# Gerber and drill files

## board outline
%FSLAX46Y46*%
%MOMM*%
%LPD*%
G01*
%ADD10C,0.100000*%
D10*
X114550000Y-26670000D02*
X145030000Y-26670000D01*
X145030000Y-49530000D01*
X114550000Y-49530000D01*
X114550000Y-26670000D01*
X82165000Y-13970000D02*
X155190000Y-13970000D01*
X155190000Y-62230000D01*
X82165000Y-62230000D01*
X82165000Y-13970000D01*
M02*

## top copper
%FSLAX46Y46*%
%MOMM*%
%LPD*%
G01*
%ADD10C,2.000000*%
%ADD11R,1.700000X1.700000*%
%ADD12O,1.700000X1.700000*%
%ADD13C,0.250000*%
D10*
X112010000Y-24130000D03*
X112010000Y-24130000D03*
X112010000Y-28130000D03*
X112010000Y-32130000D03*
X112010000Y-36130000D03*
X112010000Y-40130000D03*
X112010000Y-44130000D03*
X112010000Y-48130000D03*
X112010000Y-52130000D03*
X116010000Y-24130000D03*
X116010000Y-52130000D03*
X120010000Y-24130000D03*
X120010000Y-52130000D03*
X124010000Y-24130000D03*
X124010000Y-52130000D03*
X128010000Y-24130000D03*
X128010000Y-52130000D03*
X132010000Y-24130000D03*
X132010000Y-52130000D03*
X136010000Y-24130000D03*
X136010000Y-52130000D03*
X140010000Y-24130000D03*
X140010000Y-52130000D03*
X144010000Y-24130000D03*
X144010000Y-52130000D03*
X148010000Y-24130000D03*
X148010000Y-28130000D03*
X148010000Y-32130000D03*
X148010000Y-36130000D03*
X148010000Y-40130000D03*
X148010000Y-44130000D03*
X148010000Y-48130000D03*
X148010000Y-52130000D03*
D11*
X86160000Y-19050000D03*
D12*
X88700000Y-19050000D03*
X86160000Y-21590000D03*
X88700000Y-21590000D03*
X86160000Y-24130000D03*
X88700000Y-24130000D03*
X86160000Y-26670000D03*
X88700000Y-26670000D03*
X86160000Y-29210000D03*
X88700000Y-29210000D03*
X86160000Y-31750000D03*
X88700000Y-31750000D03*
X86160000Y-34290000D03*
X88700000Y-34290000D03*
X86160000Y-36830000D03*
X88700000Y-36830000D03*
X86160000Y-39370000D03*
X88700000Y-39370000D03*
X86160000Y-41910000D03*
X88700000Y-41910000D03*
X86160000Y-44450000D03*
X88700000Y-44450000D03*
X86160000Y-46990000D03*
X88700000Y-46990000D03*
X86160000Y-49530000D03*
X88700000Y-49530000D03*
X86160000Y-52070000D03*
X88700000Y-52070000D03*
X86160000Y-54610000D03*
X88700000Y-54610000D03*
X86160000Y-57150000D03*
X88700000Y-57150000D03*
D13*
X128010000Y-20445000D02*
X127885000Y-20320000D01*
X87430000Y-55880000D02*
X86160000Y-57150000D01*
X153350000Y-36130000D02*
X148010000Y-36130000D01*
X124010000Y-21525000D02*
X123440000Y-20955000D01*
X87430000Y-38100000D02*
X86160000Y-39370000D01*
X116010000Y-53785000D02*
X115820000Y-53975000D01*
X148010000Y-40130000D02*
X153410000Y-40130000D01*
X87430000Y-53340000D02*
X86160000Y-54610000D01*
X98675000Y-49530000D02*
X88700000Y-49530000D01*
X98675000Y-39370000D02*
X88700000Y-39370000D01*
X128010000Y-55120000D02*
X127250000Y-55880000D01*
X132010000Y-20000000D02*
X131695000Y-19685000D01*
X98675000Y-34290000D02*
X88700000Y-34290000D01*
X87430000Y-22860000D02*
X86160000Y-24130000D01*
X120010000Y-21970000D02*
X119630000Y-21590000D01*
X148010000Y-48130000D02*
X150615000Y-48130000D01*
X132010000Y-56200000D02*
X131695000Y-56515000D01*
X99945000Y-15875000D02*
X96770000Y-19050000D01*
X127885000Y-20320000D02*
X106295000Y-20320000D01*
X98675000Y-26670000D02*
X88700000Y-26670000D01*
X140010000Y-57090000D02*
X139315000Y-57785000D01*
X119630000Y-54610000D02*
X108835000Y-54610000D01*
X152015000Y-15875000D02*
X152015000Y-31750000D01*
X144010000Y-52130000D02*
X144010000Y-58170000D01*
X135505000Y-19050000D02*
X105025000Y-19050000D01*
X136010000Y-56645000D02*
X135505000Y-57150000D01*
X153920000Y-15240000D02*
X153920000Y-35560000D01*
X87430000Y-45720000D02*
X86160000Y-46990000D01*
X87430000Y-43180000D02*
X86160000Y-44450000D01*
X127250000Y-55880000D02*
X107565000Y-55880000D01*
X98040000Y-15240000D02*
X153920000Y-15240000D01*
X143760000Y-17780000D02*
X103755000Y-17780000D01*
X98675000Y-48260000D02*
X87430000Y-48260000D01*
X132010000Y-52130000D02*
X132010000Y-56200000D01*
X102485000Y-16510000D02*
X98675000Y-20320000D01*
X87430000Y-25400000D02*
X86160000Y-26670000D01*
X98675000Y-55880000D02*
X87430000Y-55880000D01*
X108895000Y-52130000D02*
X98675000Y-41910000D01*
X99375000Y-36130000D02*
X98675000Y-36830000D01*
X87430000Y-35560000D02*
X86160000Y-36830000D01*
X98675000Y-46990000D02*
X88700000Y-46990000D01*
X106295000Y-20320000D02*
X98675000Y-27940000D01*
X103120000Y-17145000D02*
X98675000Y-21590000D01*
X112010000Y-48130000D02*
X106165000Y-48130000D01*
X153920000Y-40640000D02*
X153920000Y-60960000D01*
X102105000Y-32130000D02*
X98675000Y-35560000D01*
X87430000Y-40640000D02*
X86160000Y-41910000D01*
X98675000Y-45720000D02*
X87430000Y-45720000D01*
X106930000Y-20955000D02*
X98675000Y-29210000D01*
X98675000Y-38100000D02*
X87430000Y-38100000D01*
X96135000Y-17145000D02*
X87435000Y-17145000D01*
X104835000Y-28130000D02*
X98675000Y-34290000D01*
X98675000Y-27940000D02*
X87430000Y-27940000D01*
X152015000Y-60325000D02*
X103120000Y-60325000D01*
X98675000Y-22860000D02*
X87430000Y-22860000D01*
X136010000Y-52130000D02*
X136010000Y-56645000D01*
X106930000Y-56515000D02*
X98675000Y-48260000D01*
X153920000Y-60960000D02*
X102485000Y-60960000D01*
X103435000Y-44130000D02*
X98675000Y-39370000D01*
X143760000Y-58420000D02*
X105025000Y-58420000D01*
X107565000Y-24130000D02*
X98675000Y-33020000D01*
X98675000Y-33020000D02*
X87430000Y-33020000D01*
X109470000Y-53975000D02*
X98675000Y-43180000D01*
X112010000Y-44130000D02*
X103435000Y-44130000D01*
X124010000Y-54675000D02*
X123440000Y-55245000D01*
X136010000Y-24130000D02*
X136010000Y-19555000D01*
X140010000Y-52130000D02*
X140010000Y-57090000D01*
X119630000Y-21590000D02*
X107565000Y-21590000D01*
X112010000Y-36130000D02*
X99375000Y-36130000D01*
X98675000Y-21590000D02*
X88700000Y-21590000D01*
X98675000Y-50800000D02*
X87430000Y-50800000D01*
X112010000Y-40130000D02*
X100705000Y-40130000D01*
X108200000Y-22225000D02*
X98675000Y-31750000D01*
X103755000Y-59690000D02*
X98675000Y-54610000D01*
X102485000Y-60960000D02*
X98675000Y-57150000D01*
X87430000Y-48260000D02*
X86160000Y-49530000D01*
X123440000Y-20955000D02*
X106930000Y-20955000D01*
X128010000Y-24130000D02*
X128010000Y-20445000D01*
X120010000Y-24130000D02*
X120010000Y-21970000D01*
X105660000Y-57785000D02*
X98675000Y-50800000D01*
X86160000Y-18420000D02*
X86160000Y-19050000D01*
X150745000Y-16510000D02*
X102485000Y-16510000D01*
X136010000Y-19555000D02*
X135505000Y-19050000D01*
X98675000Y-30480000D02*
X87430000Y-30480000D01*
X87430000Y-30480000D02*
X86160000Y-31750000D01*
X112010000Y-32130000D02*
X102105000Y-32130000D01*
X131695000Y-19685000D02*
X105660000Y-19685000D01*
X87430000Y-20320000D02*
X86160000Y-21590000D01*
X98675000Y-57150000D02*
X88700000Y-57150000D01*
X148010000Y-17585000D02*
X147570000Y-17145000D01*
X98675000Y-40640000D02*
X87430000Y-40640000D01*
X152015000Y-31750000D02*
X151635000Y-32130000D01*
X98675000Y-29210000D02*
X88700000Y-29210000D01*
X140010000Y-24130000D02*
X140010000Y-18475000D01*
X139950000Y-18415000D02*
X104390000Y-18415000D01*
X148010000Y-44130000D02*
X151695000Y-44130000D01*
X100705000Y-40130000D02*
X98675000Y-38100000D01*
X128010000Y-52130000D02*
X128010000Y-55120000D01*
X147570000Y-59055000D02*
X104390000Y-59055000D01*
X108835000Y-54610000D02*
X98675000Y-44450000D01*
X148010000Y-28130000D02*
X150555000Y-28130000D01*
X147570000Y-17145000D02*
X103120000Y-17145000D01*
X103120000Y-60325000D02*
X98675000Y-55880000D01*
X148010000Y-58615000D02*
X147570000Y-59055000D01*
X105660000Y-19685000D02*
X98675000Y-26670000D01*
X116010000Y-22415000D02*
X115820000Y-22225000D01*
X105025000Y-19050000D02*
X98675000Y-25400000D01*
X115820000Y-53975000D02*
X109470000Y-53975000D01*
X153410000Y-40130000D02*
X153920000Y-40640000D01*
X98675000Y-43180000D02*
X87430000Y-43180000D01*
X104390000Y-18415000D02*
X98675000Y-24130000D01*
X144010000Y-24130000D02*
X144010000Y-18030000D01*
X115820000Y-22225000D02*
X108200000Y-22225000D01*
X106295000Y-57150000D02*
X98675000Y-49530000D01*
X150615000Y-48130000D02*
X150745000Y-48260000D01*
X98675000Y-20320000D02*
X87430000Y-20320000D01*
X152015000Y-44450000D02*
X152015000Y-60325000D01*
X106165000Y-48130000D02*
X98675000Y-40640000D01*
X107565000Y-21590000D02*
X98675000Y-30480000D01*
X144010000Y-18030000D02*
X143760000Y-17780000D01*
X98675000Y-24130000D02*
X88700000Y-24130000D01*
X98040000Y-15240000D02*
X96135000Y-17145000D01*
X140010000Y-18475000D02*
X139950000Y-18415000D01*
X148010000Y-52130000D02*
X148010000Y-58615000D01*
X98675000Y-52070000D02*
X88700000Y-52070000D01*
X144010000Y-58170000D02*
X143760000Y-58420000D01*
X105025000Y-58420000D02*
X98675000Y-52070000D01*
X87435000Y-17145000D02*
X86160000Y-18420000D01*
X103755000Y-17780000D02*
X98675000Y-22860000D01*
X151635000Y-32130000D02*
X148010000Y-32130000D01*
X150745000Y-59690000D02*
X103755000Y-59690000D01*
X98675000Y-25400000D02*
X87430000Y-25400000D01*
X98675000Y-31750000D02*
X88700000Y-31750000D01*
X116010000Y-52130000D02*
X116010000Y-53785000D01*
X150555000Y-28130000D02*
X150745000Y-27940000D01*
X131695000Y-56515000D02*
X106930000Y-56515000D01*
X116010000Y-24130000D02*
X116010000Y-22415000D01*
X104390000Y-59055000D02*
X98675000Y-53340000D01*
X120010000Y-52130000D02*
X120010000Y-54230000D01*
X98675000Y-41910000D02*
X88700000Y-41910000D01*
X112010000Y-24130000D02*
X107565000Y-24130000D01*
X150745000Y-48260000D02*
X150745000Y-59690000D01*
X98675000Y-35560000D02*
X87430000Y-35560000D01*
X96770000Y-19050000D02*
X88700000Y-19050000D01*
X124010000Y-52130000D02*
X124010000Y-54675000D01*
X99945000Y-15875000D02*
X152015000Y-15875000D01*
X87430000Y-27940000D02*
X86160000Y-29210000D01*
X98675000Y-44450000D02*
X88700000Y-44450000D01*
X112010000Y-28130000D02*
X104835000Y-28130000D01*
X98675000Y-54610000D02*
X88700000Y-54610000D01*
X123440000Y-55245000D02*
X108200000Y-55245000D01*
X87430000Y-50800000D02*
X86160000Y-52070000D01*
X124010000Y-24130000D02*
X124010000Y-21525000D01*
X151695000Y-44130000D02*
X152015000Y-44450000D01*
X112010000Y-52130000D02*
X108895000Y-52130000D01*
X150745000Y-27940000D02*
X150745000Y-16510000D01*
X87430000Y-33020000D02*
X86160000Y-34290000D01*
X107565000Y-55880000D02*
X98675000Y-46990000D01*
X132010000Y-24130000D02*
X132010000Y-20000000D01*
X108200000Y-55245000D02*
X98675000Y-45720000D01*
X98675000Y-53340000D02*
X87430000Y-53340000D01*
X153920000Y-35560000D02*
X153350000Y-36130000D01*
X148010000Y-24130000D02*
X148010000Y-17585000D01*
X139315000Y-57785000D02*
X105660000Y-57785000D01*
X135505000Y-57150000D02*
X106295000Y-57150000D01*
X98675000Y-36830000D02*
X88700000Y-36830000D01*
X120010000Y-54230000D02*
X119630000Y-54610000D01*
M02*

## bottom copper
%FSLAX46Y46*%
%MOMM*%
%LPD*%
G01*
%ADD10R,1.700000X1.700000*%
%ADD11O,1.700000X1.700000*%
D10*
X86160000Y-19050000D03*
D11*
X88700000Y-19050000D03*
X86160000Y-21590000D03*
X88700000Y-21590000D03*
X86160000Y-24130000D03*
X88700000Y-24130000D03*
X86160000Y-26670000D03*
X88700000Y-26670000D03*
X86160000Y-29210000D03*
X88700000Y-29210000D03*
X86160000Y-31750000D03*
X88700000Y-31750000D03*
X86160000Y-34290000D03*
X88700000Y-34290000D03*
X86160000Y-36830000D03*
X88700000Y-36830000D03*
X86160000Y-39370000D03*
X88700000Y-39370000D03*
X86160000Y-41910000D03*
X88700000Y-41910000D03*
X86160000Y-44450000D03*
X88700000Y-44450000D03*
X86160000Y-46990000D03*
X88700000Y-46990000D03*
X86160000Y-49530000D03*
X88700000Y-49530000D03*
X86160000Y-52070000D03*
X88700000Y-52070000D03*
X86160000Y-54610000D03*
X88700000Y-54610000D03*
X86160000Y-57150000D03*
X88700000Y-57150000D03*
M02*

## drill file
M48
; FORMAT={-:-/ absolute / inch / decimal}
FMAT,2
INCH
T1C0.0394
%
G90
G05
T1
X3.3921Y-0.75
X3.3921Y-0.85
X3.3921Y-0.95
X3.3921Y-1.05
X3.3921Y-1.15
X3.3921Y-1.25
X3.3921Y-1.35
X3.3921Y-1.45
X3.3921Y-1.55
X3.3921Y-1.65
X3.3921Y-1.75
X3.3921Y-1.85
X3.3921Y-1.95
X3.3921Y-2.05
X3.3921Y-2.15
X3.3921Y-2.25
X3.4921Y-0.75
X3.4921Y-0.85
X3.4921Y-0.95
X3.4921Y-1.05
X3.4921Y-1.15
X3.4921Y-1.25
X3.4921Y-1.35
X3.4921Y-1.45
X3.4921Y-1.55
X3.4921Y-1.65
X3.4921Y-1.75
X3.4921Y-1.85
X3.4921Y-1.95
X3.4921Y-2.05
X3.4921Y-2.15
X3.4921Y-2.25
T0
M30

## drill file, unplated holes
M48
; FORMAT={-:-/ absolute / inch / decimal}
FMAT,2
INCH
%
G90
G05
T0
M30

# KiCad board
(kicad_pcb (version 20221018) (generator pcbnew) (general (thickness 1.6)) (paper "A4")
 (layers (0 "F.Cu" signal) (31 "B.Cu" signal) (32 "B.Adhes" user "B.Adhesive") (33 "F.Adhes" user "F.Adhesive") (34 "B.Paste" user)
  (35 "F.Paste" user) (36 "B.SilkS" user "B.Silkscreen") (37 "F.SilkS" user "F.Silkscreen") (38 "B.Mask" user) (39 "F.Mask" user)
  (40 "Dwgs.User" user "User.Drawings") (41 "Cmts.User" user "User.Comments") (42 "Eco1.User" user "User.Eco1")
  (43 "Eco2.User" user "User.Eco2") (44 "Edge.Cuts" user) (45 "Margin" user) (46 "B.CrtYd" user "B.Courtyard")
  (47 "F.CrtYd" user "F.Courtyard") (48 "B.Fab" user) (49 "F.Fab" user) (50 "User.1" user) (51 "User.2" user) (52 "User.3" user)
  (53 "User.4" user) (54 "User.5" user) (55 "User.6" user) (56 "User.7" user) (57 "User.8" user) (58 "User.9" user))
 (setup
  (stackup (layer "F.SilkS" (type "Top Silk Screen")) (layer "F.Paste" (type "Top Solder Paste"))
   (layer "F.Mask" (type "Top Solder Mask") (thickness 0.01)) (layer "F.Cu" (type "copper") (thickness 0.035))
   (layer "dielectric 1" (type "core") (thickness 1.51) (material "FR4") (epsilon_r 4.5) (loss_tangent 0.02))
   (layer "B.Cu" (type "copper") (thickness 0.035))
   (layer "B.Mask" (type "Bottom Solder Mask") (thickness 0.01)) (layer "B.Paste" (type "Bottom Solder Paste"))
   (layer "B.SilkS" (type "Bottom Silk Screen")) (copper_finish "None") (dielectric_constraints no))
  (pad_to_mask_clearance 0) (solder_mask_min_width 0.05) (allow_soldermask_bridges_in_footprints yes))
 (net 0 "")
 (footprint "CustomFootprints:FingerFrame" (layer "F.Cu") (at 112.01 24.13)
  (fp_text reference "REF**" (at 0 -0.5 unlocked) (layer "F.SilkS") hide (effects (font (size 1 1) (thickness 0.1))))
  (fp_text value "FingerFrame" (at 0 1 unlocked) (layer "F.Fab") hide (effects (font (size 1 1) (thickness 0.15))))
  (pad "1" smd circle (at 0 0) (size 2 2) (layers "F.Cu" "F.Paste" "F.Mask"))
  (pad "1" smd circle (at 0 0) (size 2 2) (layers "F.Cu" "F.Paste" "F.Mask"))
  (pad "1" smd circle (at 0 4) (size 2 2) (layers "F.Cu" "F.Paste" "F.Mask"))
  (pad "1" smd circle (at 0 8) (size 2 2) (layers "F.Cu" "F.Paste" "F.Mask"))
  (pad "1" smd circle (at 0 12) (size 2 2) (layers "F.Cu" "F.Paste" "F.Mask"))
  (pad "1" smd circle (at 0 16) (size 2 2) (layers "F.Cu" "F.Paste" "F.Mask"))
  (pad "1" smd circle (at 0 20) (size 2 2) (layers "F.Cu" "F.Paste" "F.Mask"))
  (pad "1" smd circle (at 0 24) (size 2 2) (layers "F.Cu" "F.Paste" "F.Mask"))
  (pad "1" smd circle (at 0 28) (size 2 2) (layers "F.Cu" "F.Paste" "F.Mask"))
  (pad "1" smd circle (at 4 0) (size 2 2) (layers "F.Cu" "F.Paste" "F.Mask"))
  (pad "1" smd circle (at 4 28) (size 2 2) (layers "F.Cu" "F.Paste" "F.Mask"))
  (pad "1" smd circle (at 8 0) (size 2 2) (layers "F.Cu" "F.Paste" "F.Mask"))
  (pad "1" smd circle (at 8 28) (size 2 2) (layers "F.Cu" "F.Paste" "F.Mask"))
  (pad "1" smd circle (at 12 0) (size 2 2) (layers "F.Cu" "F.Paste" "F.Mask"))
  (pad "1" smd circle (at 12 28) (size 2 2) (layers "F.Cu" "F.Paste" "F.Mask"))
  (pad "1" smd circle (at 16 0) (size 2 2) (layers "F.Cu" "F.Paste" "F.Mask"))
  (pad "1" smd circle (at 16 28) (size 2 2) (layers "F.Cu" "F.Paste" "F.Mask"))
  (pad "1" smd circle (at 20 0) (size 2 2) (layers "F.Cu" "F.Paste" "F.Mask"))
  (pad "1" smd circle (at 20 28) (size 2 2) (layers "F.Cu" "F.Paste" "F.Mask"))
  (pad "1" smd circle (at 24 0) (size 2 2) (layers "F.Cu" "F.Paste" "F.Mask"))
  (pad "1" smd circle (at 24 28) (size 2 2) (layers "F.Cu" "F.Paste" "F.Mask"))
  (pad "1" smd circle (at 28 0) (size 2 2) (layers "F.Cu" "F.Paste" "F.Mask"))
  (pad "1" smd circle (at 28 28) (size 2 2) (layers "F.Cu" "F.Paste" "F.Mask"))
  (pad "1" smd circle (at 32 0) (size 2 2) (layers "F.Cu" "F.Paste" "F.Mask"))
  (pad "1" smd circle (at 32 28) (size 2 2) (layers "F.Cu" "F.Paste" "F.Mask"))
  (pad "1" smd circle (at 36 0) (size 2 2) (layers "F.Cu" "F.Paste" "F.Mask"))
  (pad "1" smd circle (at 36 4) (size 2 2) (layers "F.Cu" "F.Paste" "F.Mask"))
  (pad "1" smd circle (at 36 8) (size 2 2) (layers "F.Cu" "F.Paste" "F.Mask"))
  (pad "1" smd circle (at 36 12) (size 2 2) (layers "F.Cu" "F.Paste" "F.Mask"))
  (pad "1" smd circle (at 36 16) (size 2 2) (layers "F.Cu" "F.Paste" "F.Mask"))
  (pad "1" smd circle (at 36 20) (size 2 2) (layers "F.Cu" "F.Paste" "F.Mask"))
  (pad "1" smd circle (at 36 24) (size 2 2) (layers "F.Cu" "F.Paste" "F.Mask"))
  (pad "1" smd circle (at 36 28) (size 2 2) (layers "F.Cu" "F.Paste" "F.Mask")))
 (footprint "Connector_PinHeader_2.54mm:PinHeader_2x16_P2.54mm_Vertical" (layer "F.Cu") (at 86.16 19.05)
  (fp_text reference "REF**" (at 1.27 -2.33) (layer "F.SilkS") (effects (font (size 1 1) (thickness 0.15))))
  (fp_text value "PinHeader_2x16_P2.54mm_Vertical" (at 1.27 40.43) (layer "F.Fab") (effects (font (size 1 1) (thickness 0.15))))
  (pad "1" thru_hole rect (at 0 0) (size 1.7 1.7) (drill 1) (layers "*.Cu" "*.Mask"))
  (pad "2" thru_hole oval (at 2.54 0) (size 1.7 1.7) (drill 1) (layers "*.Cu" "*.Mask"))
  (pad "3" thru_hole oval (at 0 2.54) (size 1.7 1.7) (drill 1) (layers "*.Cu" "*.Mask"))
  (pad "4" thru_hole oval (at 2.54 2.54) (size 1.7 1.7) (drill 1) (layers "*.Cu" "*.Mask"))
  (pad "5" thru_hole oval (at 0 5.08) (size 1.7 1.7) (drill 1) (layers "*.Cu" "*.Mask"))
  (pad "6" thru_hole oval (at 2.54 5.08) (size 1.7 1.7) (drill 1) (layers "*.Cu" "*.Mask"))
  (pad "7" thru_hole oval (at 0 7.62) (size 1.7 1.7) (drill 1) (layers "*.Cu" "*.Mask"))
  (pad "8" thru_hole oval (at 2.54 7.62) (size 1.7 1.7) (drill 1) (layers "*.Cu" "*.Mask"))
  (pad "9" thru_hole oval (at 0 10.16) (size 1.7 1.7) (drill 1) (layers "*.Cu" "*.Mask"))
  (pad "10" thru_hole oval (at 2.54 10.16) (size 1.7 1.7) (drill 1) (layers "*.Cu" "*.Mask"))
  (pad "11" thru_hole oval (at 0 12.7) (size 1.7 1.7) (drill 1) (layers "*.Cu" "*.Mask"))
  (pad "12" thru_hole oval (at 2.54 12.7) (size 1.7 1.7) (drill 1) (layers "*.Cu" "*.Mask"))
  (pad "13" thru_hole oval (at 0 15.24) (size 1.7 1.7) (drill 1) (layers "*.Cu" "*.Mask"))
  (pad "14" thru_hole oval (at 2.54 15.24) (size 1.7 1.7) (drill 1) (layers "*.Cu" "*.Mask"))
  (pad "15" thru_hole oval (at 0 17.78) (size 1.7 1.7) (drill 1) (layers "*.Cu" "*.Mask"))
  (pad "16" thru_hole oval (at 2.54 17.78) (size 1.7 1.7) (drill 1) (layers "*.Cu" "*.Mask"))
  (pad "17" thru_hole oval (at 0 20.32) (size 1.7 1.7) (drill 1) (layers "*.Cu" "*.Mask"))
  (pad "18" thru_hole oval (at 2.54 20.32) (size 1.7 1.7) (drill 1) (layers "*.Cu" "*.Mask"))
  (pad "19" thru_hole oval (at 0 22.86) (size 1.7 1.7) (drill 1) (layers "*.Cu" "*.Mask"))
  (pad "20" thru_hole oval (at 2.54 22.86) (size 1.7 1.7) (drill 1) (layers "*.Cu" "*.Mask"))
  (pad "21" thru_hole oval (at 0 25.4) (size 1.7 1.7) (drill 1) (layers "*.Cu" "*.Mask"))
  (pad "22" thru_hole oval (at 2.54 25.4) (size 1.7 1.7) (drill 1) (layers "*.Cu" "*.Mask"))
  (pad "23" thru_hole oval (at 0 27.94) (size 1.7 1.7) (drill 1) (layers "*.Cu" "*.Mask"))
  (pad "24" thru_hole oval (at 2.54 27.94) (size 1.7 1.7) (drill 1) (layers "*.Cu" "*.Mask"))
  (pad "25" thru_hole oval (at 0 30.48) (size 1.7 1.7) (drill 1) (layers "*.Cu" "*.Mask"))
  (pad "26" thru_hole oval (at 2.54 30.48) (size 1.7 1.7) (drill 1) (layers "*.Cu" "*.Mask"))
  (pad "27" thru_hole oval (at 0 33.02) (size 1.7 1.7) (drill 1) (layers "*.Cu" "*.Mask"))
  (pad "28" thru_hole oval (at 2.54 33.02) (size 1.7 1.7) (drill 1) (layers "*.Cu" "*.Mask"))
  (pad "29" thru_hole oval (at 0 35.56) (size 1.7 1.7) (drill 1) (layers "*.Cu" "*.Mask"))
  (pad "30" thru_hole oval (at 2.54 35.56) (size 1.7 1.7) (drill 1) (layers "*.Cu" "*.Mask"))
  (pad "31" thru_hole oval (at 0 38.1) (size 1.7 1.7) (drill 1) (layers "*.Cu" "*.Mask"))
  (pad "32" thru_hole oval (at 2.54 38.1) (size 1.7 1.7) (drill 1) (layers "*.Cu" "*.Mask")))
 (gr_rect (start 114.55 26.67) (end 145.03 49.53) (stroke (width 0.1) (type default)) (fill none) (layer "Edge.Cuts"))
 (gr_rect (start 82.165 13.97) (end 155.19 62.23) (stroke (width 0.1) (type default)) (fill none) (layer "Edge.Cuts"))
 (segment (start 128.01 20.445) (end 127.885 20.32) (width 0.25) (layer "F.Cu") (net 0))
 (segment (start 87.43 55.88) (end 86.16 57.15) (width 0.25) (layer "F.Cu") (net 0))
 (segment (start 153.35 36.13) (end 148.01 36.13) (width 0.25) (layer "F.Cu") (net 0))
 (segment (start 124.01 21.525) (end 123.44 20.955) (width 0.25) (layer "F.Cu") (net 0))
 (segment (start 87.43 38.1) (end 86.16 39.37) (width 0.25) (layer "F.Cu") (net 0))
 (segment (start 116.01 53.785) (end 115.82 53.975) (width 0.25) (layer "F.Cu") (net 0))
 (segment (start 148.01 40.13) (end 153.41 40.13) (width 0.25) (layer "F.Cu") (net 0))
 (segment (start 87.43 53.34) (end 86.16 54.61) (width 0.25) (layer "F.Cu") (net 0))
 (segment (start 98.675 49.53) (end 88.7 49.53) (width 0.25) (layer "F.Cu") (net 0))
 (segment (start 98.675 39.37) (end 88.7 39.37) (width 0.25) (layer "F.Cu") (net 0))
 (segment (start 128.01 55.12) (end 127.25 55.88) (width 0.25) (layer "F.Cu") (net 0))
 (segment (start 132.01 20) (end 131.695 19.685) (width 0.25) (layer "F.Cu") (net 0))
 (segment (start 98.675 34.29) (end 88.7 34.29) (width 0.25) (layer "F.Cu") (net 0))
 (segment (start 87.43 22.86) (end 86.16 24.13) (width 0.25) (layer "F.Cu") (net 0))
 (segment (start 120.01 21.97) (end 119.63 21.59) (width 0.25) (layer "F.Cu") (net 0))
 (segment (start 148.01 48.13) (end 150.615 48.13) (width 0.25) (layer "F.Cu") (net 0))
 (segment (start 132.01 56.2) (end 131.695 56.515) (width 0.25) (layer "F.Cu") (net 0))
 (segment (start 99.945 15.875) (end 96.77 19.05) (width 0.25) (layer "F.Cu") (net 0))
 (segment (start 127.885 20.32) (end 106.295 20.32) (width 0.25) (layer "F.Cu") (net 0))
 (segment (start 98.675 26.67) (end 88.7 26.67) (width 0.25) (layer "F.Cu") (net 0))
 (segment (start 140.01 57.09) (end 139.315 57.785) (width 0.25) (layer "F.Cu") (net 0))
 (segment (start 119.63 54.61) (end 108.835 54.61) (width 0.25) (layer "F.Cu") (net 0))
 (segment (start 152.015 15.875) (end 152.015 31.75) (width 0.25) (layer "F.Cu") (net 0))
 (segment (start 144.01 52.13) (end 144.01 58.17) (width 0.25) (layer "F.Cu") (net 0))
 (segment (start 135.505 19.05) (end 105.025 19.05) (width 0.25) (layer "F.Cu") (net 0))
 (segment (start 136.01 56.645) (end 135.505 57.15) (width 0.25) (layer "F.Cu") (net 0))
 (segment (start 153.92 15.24) (end 153.92 35.56) (width 0.25) (layer "F.Cu") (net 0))
 (segment (start 87.43 45.72) (end 86.16 46.99) (width 0.25) (layer "F.Cu") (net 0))
 (segment (start 87.43 43.18) (end 86.16 44.45) (width 0.25) (layer "F.Cu") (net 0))
 (segment (start 127.25 55.88) (end 107.565 55.88) (width 0.25) (layer "F.Cu") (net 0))
 (segment (start 98.04 15.24) (end 153.92 15.24) (width 0.25) (layer "F.Cu") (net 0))
 (segment (start 143.76 17.78) (end 103.755 17.78) (width 0.25) (layer "F.Cu") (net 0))
 (segment (start 98.675 48.26) (end 87.43 48.26) (width 0.25) (layer "F.Cu") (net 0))
 (segment (start 132.01 52.13) (end 132.01 56.2) (width 0.25) (layer "F.Cu") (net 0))
 (segment (start 102.485 16.51) (end 98.675 20.32) (width 0.25) (layer "F.Cu") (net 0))
 (segment (start 87.43 25.4) (end 86.16 26.67) (width 0.25) (layer "F.Cu") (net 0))
 (segment (start 98.675 55.88) (end 87.43 55.88) (width 0.25) (layer "F.Cu") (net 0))
 (segment (start 108.895 52.13) (end 98.675 41.91) (width 0.25) (layer "F.Cu") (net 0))
 (segment (start 99.375 36.13) (end 98.675 36.83) (width 0.25) (layer "F.Cu") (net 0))
 (segment (start 87.43 35.56) (end 86.16 36.83) (width 0.25) (layer "F.Cu") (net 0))
 (segment (start 98.675 46.99) (end 88.7 46.99) (width 0.25) (layer "F.Cu") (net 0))
 (segment (start 106.295 20.32) (end 98.675 27.94) (width 0.25) (layer "F.Cu") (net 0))
 (segment (start 103.12 17.145) (end 98.675 21.59) (width 0.25) (layer "F.Cu") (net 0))
 (segment (start 112.01 48.13) (end 106.165 48.13) (width 0.25) (layer "F.Cu") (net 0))
 (segment (start 153.92 40.64) (end 153.92 60.96) (width 0.25) (layer "F.Cu") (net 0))
 (segment (start 102.105 32.13) (end 98.675 35.56) (width 0.25) (layer "F.Cu") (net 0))
 (segment (start 87.43 40.64) (end 86.16 41.91) (width 0.25) (layer "F.Cu") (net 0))
 (segment (start 98.675 45.72) (end 87.43 45.72) (width 0.25) (layer "F.Cu") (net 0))
 (segment (start 106.93 20.955) (end 98.675 29.21) (width 0.25) (layer "F.Cu") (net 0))
 (segment (start 98.675 38.1) (end 87.43 38.1) (width 0.25) (layer "F.Cu") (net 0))
 (segment (start 96.135 17.145) (end 87.435 17.145) (width 0.25) (layer "F.Cu") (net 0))
 (segment (start 104.835 28.13) (end 98.675 34.29) (width 0.25) (layer "F.Cu") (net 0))
 (segment (start 98.675 27.94) (end 87.43 27.94) (width 0.25) (layer "F.Cu") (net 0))
 (segment (start 152.015 60.325) (end 103.12 60.325) (width 0.25) (layer "F.Cu") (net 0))
 (segment (start 98.675 22.86) (end 87.43 22.86) (width 0.25) (layer "F.Cu") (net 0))
 (segment (start 136.01 52.13) (end 136.01 56.645) (width 0.25) (layer "F.Cu") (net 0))
 (segment (start 106.93 56.515) (end 98.675 48.26) (width 0.25) (layer "F.Cu") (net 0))
 (segment (start 153.92 60.96) (end 102.485 60.96) (width 0.25) (layer "F.Cu") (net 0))
 (segment (start 103.435 44.13) (end 98.675 39.37) (width 0.25) (layer "F.Cu") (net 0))
 (segment (start 143.76 58.42) (end 105.025 58.42) (width 0.25) (layer "F.Cu") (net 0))
 (segment (start 107.565 24.13) (end 98.675 33.02) (width 0.25) (layer "F.Cu") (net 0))
 (segment (start 98.675 33.02) (end 87.43 33.02) (width 0.25) (layer "F.Cu") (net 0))
 (segment (start 109.47 53.975) (end 98.675 43.18) (width 0.25) (layer "F.Cu") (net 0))
 (segment (start 112.01 44.13) (end 103.435 44.13) (width 0.25) (layer "F.Cu") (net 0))
 (segment (start 124.01 54.675) (end 123.44 55.245) (width 0.25) (layer "F.Cu") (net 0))
 (segment (start 136.01 24.13) (end 136.01 19.555) (width 0.25) (layer "F.Cu") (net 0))
 (segment (start 140.01 52.13) (end 140.01 57.09) (width 0.25) (layer "F.Cu") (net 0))
 (segment (start 119.63 21.59) (end 107.565 21.59) (width 0.25) (layer "F.Cu") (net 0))
 (segment (start 112.01 36.13) (end 99.375 36.13) (width 0.25) (layer "F.Cu") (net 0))
 (segment (start 98.675 21.59) (end 88.7 21.59) (width 0.25) (layer "F.Cu") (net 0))
 (segment (start 98.675 50.8) (end 87.43 50.8) (width 0.25) (layer "F.Cu") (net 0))
 (segment (start 112.01 40.13) (end 100.705 40.13) (width 0.25) (layer "F.Cu") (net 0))
 (segment (start 108.2 22.225) (end 98.675 31.75) (width 0.25) (layer "F.Cu") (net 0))
 (segment (start 103.755 59.69) (end 98.675 54.61) (width 0.25) (layer "F.Cu") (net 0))
 (segment (start 102.485 60.96) (end 98.675 57.15) (width 0.25) (layer "F.Cu") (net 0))
 (segment (start 87.43 48.26) (end 86.16 49.53) (width 0.25) (layer "F.Cu") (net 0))
 (segment (start 123.44 20.955) (end 106.93 20.955) (width 0.25) (layer "F.Cu") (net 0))
 (segment (start 128.01 24.13) (end 128.01 20.445) (width 0.25) (layer "F.Cu") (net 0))
 (segment (start 120.01 24.13) (end 120.01 21.97) (width 0.25) (layer "F.Cu") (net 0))
 (segment (start 105.66 57.785) (end 98.675 50.8) (width 0.25) (layer "F.Cu") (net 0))
 (segment (start 86.16 18.42) (end 86.16 19.05) (width 0.25) (layer "F.Cu") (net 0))
 (segment (start 150.745 16.51) (end 102.485 16.51) (width 0.25) (layer "F.Cu") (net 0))
 (segment (start 136.01 19.555) (end 135.505 19.05) (width 0.25) (layer "F.Cu") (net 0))
 (segment (start 98.675 30.48) (end 87.43 30.48) (width 0.25) (layer "F.Cu") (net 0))
 (segment (start 87.43 30.48) (end 86.16 31.75) (width 0.25) (layer "F.Cu") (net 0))
 (segment (start 112.01 32.13) (end 102.105 32.13) (width 0.25) (layer "F.Cu") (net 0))
 (segment (start 131.695 19.685) (end 105.66 19.685) (width 0.25) (layer "F.Cu") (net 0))
 (segment (start 87.43 20.32) (end 86.16 21.59) (width 0.25) (layer "F.Cu") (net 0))
 (segment (start 98.675 57.15) (end 88.7 57.15) (width 0.25) (layer "F.Cu") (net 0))
 (segment (start 148.01 17.585) (end 147.57 17.145) (width 0.25) (layer "F.Cu") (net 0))
 (segment (start 98.675 40.64) (end 87.43 40.64) (width 0.25) (layer "F.Cu") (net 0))
 (segment (start 152.015 31.75) (end 151.635 32.13) (width 0.25) (layer "F.Cu") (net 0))
 (segment (start 98.675 29.21) (end 88.7 29.21) (width 0.25) (layer "F.Cu") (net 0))
 (segment (start 140.01 24.13) (end 140.01 18.475) (width 0.25) (layer "F.Cu") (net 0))
 (segment (start 139.95 18.415) (end 104.39 18.415) (width 0.25) (layer "F.Cu") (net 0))
 (segment (start 148.01 44.13) (end 151.695 44.13) (width 0.25) (layer "F.Cu") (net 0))
 (segment (start 100.705 40.13) (end 98.675 38.1) (width 0.25) (layer "F.Cu") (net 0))
 (segment (start 128.01 52.13) (end 128.01 55.12) (width 0.25) (layer "F.Cu") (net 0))
 (segment (start 147.57 59.055) (end 104.39 59.055) (width 0.25) (layer "F.Cu") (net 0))
 (segment (start 108.835 54.61) (end 98.675 44.45) (width 0.25) (layer "F.Cu") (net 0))
 (segment (start 148.01 28.13) (end 150.555 28.13) (width 0.25) (layer "F.Cu") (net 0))
 (segment (start 147.57 17.145) (end 103.12 17.145) (width 0.25) (layer "F.Cu") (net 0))
 (segment (start 103.12 60.325) (end 98.675 55.88) (width 0.25) (layer "F.Cu") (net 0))
 (segment (start 148.01 58.615) (end 147.57 59.055) (width 0.25) (layer "F.Cu") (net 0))
 (segment (start 105.66 19.685) (end 98.675 26.67) (width 0.25) (layer "F.Cu") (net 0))
 (segment (start 116.01 22.415) (end 115.82 22.225) (width 0.25) (layer "F.Cu") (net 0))
 (segment (start 105.025 19.05) (end 98.675 25.4) (width 0.25) (layer "F.Cu") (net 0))
 (segment (start 115.82 53.975) (end 109.47 53.975) (width 0.25) (layer "F.Cu") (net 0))
 (segment (start 153.41 40.13) (end 153.92 40.64) (width 0.25) (layer "F.Cu") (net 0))
 (segment (start 98.675 43.18) (end 87.43 43.18) (width 0.25) (layer "F.Cu") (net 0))
 (segment (start 104.39 18.415) (end 98.675 24.13) (width 0.25) (layer "F.Cu") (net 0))
 (segment (start 144.01 24.13) (end 144.01 18.03) (width 0.25) (layer "F.Cu") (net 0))
 (segment (start 115.82 22.225) (end 108.2 22.225) (width 0.25) (layer "F.Cu") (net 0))
 (segment (start 106.295 57.15) (end 98.675 49.53) (width 0.25) (layer "F.Cu") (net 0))
 (segment (start 150.615 48.13) (end 150.745 48.26) (width 0.25) (layer "F.Cu") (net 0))
 (segment (start 98.675 20.32) (end 87.43 20.32) (width 0.25) (layer "F.Cu") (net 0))
 (segment (start 152.015 44.45) (end 152.015 60.325) (width 0.25) (layer "F.Cu") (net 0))
 (segment (start 106.165 48.13) (end 98.675 40.64) (width 0.25) (layer "F.Cu") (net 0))
 (segment (start 107.565 21.59) (end 98.675 30.48) (width 0.25) (layer "F.Cu") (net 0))
 (segment (start 144.01 18.03) (end 143.76 17.78) (width 0.25) (layer "F.Cu") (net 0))
 (segment (start 98.675 24.13) (end 88.7 24.13) (width 0.25) (layer "F.Cu") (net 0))
 (segment (start 98.04 15.24) (end 96.135 17.145) (width 0.25) (layer "F.Cu") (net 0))
 (segment (start 140.01 18.475) (end 139.95 18.415) (width 0.25) (layer "F.Cu") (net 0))
 (segment (start 148.01 52.13) (end 148.01 58.615) (width 0.25) (layer "F.Cu") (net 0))
 (segment (start 98.675 52.07) (end 88.7 52.07) (width 0.25) (layer "F.Cu") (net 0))
 (segment (start 144.01 58.17) (end 143.76 58.42) (width 0.25) (layer "F.Cu") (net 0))
 (segment (start 105.025 58.42) (end 98.675 52.07) (width 0.25) (layer "F.Cu") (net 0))
 (segment (start 87.435 17.145) (end 86.16 18.42) (width 0.25) (layer "F.Cu") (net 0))
 (segment (start 103.755 17.78) (end 98.675 22.86) (width 0.25) (layer "F.Cu") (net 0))
 (segment (start 151.635 32.13) (end 148.01 32.13) (width 0.25) (layer "F.Cu") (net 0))
 (segment (start 150.745 59.69) (end 103.755 59.69) (width 0.25) (layer "F.Cu") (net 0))
 (segment (start 98.675 25.4) (end 87.43 25.4) (width 0.25) (layer "F.Cu") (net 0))
 (segment (start 98.675 31.75) (end 88.7 31.75) (width 0.25) (layer "F.Cu") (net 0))
 (segment (start 116.01 52.13) (end 116.01 53.785) (width 0.25) (layer "F.Cu") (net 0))
 (segment (start 150.555 28.13) (end 150.745 27.94) (width 0.25) (layer "F.Cu") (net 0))
 (segment (start 131.695 56.515) (end 106.93 56.515) (width 0.25) (layer "F.Cu") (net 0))
 (segment (start 116.01 24.13) (end 116.01 22.415) (width 0.25) (layer "F.Cu") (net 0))
 (segment (start 104.39 59.055) (end 98.675 53.34) (width 0.25) (layer "F.Cu") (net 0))
 (segment (start 120.01 52.13) (end 120.01 54.23) (width 0.25) (layer "F.Cu") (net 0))
 (segment (start 98.675 41.91) (end 88.7 41.91) (width 0.25) (layer "F.Cu") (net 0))
 (segment (start 112.01 24.13) (end 107.565 24.13) (width 0.25) (layer "F.Cu") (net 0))
 (segment (start 150.745 48.26) (end 150.745 59.69) (width 0.25) (layer "F.Cu") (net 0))
 (segment (start 98.675 35.56) (end 87.43 35.56) (width 0.25) (layer "F.Cu") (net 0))
 (segment (start 96.77 19.05) (end 88.7 19.05) (width 0.25) (layer "F.Cu") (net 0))
 (segment (start 124.01 52.13) (end 124.01 54.675) (width 0.25) (layer "F.Cu") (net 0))
 (segment (start 99.945 15.875) (end 152.015 15.875) (width 0.25) (layer "F.Cu") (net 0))
 (segment (start 87.43 27.94) (end 86.16 29.21) (width 0.25) (layer "F.Cu") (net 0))
 (segment (start 98.675 44.45) (end 88.7 44.45) (width 0.25) (layer "F.Cu") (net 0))
 (segment (start 112.01 28.13) (end 104.835 28.13) (width 0.25) (layer "F.Cu") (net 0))
 (segment (start 98.675 54.61) (end 88.7 54.61) (width 0.25) (layer "F.Cu") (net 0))
 (segment (start 123.44 55.245) (end 108.2 55.245) (width 0.25) (layer "F.Cu") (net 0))
 (segment (start 87.43 50.8) (end 86.16 52.07) (width 0.25) (layer "F.Cu") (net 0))
 (segment (start 124.01 24.13) (end 124.01 21.525) (width 0.25) (layer "F.Cu") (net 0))
 (segment (start 151.695 44.13) (end 152.015 44.45) (width 0.25) (layer "F.Cu") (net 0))
 (segment (start 112.01 52.13) (end 108.895 52.13) (width 0.25) (layer "F.Cu") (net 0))
 (segment (start 150.745 27.94) (end 150.745 16.51) (width 0.25) (layer "F.Cu") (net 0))
 (segment (start 87.43 33.02) (end 86.16 34.29) (width 0.25) (layer "F.Cu") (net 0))
 (segment (start 107.565 55.88) (end 98.675 46.99) (width 0.25) (layer "F.Cu") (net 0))
 (segment (start 132.01 24.13) (end 132.01 20) (width 0.25) (layer "F.Cu") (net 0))
 (segment (start 108.2 55.245) (end 98.675 45.72) (width 0.25) (layer "F.Cu") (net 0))
 (segment (start 98.675 53.34) (end 87.43 53.34) (width 0.25) (layer "F.Cu") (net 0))
 (segment (start 153.92 35.56) (end 153.35 36.13) (width 0.25) (layer "F.Cu") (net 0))
 (segment (start 148.01 24.13) (end 148.01 17.585) (width 0.25) (layer "F.Cu") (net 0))
 (segment (start 139.315 57.785) (end 105.66 57.785) (width 0.25) (layer "F.Cu") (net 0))
 (segment (start 135.505 57.15) (end 106.295 57.15) (width 0.25) (layer "F.Cu") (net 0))
 (segment (start 98.675 36.83) (end 88.7 36.83) (width 0.25) (layer "F.Cu") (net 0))
 (segment (start 120.01 54.23) (end 119.63 54.61) (width 0.25) (layer "F.Cu") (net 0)))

